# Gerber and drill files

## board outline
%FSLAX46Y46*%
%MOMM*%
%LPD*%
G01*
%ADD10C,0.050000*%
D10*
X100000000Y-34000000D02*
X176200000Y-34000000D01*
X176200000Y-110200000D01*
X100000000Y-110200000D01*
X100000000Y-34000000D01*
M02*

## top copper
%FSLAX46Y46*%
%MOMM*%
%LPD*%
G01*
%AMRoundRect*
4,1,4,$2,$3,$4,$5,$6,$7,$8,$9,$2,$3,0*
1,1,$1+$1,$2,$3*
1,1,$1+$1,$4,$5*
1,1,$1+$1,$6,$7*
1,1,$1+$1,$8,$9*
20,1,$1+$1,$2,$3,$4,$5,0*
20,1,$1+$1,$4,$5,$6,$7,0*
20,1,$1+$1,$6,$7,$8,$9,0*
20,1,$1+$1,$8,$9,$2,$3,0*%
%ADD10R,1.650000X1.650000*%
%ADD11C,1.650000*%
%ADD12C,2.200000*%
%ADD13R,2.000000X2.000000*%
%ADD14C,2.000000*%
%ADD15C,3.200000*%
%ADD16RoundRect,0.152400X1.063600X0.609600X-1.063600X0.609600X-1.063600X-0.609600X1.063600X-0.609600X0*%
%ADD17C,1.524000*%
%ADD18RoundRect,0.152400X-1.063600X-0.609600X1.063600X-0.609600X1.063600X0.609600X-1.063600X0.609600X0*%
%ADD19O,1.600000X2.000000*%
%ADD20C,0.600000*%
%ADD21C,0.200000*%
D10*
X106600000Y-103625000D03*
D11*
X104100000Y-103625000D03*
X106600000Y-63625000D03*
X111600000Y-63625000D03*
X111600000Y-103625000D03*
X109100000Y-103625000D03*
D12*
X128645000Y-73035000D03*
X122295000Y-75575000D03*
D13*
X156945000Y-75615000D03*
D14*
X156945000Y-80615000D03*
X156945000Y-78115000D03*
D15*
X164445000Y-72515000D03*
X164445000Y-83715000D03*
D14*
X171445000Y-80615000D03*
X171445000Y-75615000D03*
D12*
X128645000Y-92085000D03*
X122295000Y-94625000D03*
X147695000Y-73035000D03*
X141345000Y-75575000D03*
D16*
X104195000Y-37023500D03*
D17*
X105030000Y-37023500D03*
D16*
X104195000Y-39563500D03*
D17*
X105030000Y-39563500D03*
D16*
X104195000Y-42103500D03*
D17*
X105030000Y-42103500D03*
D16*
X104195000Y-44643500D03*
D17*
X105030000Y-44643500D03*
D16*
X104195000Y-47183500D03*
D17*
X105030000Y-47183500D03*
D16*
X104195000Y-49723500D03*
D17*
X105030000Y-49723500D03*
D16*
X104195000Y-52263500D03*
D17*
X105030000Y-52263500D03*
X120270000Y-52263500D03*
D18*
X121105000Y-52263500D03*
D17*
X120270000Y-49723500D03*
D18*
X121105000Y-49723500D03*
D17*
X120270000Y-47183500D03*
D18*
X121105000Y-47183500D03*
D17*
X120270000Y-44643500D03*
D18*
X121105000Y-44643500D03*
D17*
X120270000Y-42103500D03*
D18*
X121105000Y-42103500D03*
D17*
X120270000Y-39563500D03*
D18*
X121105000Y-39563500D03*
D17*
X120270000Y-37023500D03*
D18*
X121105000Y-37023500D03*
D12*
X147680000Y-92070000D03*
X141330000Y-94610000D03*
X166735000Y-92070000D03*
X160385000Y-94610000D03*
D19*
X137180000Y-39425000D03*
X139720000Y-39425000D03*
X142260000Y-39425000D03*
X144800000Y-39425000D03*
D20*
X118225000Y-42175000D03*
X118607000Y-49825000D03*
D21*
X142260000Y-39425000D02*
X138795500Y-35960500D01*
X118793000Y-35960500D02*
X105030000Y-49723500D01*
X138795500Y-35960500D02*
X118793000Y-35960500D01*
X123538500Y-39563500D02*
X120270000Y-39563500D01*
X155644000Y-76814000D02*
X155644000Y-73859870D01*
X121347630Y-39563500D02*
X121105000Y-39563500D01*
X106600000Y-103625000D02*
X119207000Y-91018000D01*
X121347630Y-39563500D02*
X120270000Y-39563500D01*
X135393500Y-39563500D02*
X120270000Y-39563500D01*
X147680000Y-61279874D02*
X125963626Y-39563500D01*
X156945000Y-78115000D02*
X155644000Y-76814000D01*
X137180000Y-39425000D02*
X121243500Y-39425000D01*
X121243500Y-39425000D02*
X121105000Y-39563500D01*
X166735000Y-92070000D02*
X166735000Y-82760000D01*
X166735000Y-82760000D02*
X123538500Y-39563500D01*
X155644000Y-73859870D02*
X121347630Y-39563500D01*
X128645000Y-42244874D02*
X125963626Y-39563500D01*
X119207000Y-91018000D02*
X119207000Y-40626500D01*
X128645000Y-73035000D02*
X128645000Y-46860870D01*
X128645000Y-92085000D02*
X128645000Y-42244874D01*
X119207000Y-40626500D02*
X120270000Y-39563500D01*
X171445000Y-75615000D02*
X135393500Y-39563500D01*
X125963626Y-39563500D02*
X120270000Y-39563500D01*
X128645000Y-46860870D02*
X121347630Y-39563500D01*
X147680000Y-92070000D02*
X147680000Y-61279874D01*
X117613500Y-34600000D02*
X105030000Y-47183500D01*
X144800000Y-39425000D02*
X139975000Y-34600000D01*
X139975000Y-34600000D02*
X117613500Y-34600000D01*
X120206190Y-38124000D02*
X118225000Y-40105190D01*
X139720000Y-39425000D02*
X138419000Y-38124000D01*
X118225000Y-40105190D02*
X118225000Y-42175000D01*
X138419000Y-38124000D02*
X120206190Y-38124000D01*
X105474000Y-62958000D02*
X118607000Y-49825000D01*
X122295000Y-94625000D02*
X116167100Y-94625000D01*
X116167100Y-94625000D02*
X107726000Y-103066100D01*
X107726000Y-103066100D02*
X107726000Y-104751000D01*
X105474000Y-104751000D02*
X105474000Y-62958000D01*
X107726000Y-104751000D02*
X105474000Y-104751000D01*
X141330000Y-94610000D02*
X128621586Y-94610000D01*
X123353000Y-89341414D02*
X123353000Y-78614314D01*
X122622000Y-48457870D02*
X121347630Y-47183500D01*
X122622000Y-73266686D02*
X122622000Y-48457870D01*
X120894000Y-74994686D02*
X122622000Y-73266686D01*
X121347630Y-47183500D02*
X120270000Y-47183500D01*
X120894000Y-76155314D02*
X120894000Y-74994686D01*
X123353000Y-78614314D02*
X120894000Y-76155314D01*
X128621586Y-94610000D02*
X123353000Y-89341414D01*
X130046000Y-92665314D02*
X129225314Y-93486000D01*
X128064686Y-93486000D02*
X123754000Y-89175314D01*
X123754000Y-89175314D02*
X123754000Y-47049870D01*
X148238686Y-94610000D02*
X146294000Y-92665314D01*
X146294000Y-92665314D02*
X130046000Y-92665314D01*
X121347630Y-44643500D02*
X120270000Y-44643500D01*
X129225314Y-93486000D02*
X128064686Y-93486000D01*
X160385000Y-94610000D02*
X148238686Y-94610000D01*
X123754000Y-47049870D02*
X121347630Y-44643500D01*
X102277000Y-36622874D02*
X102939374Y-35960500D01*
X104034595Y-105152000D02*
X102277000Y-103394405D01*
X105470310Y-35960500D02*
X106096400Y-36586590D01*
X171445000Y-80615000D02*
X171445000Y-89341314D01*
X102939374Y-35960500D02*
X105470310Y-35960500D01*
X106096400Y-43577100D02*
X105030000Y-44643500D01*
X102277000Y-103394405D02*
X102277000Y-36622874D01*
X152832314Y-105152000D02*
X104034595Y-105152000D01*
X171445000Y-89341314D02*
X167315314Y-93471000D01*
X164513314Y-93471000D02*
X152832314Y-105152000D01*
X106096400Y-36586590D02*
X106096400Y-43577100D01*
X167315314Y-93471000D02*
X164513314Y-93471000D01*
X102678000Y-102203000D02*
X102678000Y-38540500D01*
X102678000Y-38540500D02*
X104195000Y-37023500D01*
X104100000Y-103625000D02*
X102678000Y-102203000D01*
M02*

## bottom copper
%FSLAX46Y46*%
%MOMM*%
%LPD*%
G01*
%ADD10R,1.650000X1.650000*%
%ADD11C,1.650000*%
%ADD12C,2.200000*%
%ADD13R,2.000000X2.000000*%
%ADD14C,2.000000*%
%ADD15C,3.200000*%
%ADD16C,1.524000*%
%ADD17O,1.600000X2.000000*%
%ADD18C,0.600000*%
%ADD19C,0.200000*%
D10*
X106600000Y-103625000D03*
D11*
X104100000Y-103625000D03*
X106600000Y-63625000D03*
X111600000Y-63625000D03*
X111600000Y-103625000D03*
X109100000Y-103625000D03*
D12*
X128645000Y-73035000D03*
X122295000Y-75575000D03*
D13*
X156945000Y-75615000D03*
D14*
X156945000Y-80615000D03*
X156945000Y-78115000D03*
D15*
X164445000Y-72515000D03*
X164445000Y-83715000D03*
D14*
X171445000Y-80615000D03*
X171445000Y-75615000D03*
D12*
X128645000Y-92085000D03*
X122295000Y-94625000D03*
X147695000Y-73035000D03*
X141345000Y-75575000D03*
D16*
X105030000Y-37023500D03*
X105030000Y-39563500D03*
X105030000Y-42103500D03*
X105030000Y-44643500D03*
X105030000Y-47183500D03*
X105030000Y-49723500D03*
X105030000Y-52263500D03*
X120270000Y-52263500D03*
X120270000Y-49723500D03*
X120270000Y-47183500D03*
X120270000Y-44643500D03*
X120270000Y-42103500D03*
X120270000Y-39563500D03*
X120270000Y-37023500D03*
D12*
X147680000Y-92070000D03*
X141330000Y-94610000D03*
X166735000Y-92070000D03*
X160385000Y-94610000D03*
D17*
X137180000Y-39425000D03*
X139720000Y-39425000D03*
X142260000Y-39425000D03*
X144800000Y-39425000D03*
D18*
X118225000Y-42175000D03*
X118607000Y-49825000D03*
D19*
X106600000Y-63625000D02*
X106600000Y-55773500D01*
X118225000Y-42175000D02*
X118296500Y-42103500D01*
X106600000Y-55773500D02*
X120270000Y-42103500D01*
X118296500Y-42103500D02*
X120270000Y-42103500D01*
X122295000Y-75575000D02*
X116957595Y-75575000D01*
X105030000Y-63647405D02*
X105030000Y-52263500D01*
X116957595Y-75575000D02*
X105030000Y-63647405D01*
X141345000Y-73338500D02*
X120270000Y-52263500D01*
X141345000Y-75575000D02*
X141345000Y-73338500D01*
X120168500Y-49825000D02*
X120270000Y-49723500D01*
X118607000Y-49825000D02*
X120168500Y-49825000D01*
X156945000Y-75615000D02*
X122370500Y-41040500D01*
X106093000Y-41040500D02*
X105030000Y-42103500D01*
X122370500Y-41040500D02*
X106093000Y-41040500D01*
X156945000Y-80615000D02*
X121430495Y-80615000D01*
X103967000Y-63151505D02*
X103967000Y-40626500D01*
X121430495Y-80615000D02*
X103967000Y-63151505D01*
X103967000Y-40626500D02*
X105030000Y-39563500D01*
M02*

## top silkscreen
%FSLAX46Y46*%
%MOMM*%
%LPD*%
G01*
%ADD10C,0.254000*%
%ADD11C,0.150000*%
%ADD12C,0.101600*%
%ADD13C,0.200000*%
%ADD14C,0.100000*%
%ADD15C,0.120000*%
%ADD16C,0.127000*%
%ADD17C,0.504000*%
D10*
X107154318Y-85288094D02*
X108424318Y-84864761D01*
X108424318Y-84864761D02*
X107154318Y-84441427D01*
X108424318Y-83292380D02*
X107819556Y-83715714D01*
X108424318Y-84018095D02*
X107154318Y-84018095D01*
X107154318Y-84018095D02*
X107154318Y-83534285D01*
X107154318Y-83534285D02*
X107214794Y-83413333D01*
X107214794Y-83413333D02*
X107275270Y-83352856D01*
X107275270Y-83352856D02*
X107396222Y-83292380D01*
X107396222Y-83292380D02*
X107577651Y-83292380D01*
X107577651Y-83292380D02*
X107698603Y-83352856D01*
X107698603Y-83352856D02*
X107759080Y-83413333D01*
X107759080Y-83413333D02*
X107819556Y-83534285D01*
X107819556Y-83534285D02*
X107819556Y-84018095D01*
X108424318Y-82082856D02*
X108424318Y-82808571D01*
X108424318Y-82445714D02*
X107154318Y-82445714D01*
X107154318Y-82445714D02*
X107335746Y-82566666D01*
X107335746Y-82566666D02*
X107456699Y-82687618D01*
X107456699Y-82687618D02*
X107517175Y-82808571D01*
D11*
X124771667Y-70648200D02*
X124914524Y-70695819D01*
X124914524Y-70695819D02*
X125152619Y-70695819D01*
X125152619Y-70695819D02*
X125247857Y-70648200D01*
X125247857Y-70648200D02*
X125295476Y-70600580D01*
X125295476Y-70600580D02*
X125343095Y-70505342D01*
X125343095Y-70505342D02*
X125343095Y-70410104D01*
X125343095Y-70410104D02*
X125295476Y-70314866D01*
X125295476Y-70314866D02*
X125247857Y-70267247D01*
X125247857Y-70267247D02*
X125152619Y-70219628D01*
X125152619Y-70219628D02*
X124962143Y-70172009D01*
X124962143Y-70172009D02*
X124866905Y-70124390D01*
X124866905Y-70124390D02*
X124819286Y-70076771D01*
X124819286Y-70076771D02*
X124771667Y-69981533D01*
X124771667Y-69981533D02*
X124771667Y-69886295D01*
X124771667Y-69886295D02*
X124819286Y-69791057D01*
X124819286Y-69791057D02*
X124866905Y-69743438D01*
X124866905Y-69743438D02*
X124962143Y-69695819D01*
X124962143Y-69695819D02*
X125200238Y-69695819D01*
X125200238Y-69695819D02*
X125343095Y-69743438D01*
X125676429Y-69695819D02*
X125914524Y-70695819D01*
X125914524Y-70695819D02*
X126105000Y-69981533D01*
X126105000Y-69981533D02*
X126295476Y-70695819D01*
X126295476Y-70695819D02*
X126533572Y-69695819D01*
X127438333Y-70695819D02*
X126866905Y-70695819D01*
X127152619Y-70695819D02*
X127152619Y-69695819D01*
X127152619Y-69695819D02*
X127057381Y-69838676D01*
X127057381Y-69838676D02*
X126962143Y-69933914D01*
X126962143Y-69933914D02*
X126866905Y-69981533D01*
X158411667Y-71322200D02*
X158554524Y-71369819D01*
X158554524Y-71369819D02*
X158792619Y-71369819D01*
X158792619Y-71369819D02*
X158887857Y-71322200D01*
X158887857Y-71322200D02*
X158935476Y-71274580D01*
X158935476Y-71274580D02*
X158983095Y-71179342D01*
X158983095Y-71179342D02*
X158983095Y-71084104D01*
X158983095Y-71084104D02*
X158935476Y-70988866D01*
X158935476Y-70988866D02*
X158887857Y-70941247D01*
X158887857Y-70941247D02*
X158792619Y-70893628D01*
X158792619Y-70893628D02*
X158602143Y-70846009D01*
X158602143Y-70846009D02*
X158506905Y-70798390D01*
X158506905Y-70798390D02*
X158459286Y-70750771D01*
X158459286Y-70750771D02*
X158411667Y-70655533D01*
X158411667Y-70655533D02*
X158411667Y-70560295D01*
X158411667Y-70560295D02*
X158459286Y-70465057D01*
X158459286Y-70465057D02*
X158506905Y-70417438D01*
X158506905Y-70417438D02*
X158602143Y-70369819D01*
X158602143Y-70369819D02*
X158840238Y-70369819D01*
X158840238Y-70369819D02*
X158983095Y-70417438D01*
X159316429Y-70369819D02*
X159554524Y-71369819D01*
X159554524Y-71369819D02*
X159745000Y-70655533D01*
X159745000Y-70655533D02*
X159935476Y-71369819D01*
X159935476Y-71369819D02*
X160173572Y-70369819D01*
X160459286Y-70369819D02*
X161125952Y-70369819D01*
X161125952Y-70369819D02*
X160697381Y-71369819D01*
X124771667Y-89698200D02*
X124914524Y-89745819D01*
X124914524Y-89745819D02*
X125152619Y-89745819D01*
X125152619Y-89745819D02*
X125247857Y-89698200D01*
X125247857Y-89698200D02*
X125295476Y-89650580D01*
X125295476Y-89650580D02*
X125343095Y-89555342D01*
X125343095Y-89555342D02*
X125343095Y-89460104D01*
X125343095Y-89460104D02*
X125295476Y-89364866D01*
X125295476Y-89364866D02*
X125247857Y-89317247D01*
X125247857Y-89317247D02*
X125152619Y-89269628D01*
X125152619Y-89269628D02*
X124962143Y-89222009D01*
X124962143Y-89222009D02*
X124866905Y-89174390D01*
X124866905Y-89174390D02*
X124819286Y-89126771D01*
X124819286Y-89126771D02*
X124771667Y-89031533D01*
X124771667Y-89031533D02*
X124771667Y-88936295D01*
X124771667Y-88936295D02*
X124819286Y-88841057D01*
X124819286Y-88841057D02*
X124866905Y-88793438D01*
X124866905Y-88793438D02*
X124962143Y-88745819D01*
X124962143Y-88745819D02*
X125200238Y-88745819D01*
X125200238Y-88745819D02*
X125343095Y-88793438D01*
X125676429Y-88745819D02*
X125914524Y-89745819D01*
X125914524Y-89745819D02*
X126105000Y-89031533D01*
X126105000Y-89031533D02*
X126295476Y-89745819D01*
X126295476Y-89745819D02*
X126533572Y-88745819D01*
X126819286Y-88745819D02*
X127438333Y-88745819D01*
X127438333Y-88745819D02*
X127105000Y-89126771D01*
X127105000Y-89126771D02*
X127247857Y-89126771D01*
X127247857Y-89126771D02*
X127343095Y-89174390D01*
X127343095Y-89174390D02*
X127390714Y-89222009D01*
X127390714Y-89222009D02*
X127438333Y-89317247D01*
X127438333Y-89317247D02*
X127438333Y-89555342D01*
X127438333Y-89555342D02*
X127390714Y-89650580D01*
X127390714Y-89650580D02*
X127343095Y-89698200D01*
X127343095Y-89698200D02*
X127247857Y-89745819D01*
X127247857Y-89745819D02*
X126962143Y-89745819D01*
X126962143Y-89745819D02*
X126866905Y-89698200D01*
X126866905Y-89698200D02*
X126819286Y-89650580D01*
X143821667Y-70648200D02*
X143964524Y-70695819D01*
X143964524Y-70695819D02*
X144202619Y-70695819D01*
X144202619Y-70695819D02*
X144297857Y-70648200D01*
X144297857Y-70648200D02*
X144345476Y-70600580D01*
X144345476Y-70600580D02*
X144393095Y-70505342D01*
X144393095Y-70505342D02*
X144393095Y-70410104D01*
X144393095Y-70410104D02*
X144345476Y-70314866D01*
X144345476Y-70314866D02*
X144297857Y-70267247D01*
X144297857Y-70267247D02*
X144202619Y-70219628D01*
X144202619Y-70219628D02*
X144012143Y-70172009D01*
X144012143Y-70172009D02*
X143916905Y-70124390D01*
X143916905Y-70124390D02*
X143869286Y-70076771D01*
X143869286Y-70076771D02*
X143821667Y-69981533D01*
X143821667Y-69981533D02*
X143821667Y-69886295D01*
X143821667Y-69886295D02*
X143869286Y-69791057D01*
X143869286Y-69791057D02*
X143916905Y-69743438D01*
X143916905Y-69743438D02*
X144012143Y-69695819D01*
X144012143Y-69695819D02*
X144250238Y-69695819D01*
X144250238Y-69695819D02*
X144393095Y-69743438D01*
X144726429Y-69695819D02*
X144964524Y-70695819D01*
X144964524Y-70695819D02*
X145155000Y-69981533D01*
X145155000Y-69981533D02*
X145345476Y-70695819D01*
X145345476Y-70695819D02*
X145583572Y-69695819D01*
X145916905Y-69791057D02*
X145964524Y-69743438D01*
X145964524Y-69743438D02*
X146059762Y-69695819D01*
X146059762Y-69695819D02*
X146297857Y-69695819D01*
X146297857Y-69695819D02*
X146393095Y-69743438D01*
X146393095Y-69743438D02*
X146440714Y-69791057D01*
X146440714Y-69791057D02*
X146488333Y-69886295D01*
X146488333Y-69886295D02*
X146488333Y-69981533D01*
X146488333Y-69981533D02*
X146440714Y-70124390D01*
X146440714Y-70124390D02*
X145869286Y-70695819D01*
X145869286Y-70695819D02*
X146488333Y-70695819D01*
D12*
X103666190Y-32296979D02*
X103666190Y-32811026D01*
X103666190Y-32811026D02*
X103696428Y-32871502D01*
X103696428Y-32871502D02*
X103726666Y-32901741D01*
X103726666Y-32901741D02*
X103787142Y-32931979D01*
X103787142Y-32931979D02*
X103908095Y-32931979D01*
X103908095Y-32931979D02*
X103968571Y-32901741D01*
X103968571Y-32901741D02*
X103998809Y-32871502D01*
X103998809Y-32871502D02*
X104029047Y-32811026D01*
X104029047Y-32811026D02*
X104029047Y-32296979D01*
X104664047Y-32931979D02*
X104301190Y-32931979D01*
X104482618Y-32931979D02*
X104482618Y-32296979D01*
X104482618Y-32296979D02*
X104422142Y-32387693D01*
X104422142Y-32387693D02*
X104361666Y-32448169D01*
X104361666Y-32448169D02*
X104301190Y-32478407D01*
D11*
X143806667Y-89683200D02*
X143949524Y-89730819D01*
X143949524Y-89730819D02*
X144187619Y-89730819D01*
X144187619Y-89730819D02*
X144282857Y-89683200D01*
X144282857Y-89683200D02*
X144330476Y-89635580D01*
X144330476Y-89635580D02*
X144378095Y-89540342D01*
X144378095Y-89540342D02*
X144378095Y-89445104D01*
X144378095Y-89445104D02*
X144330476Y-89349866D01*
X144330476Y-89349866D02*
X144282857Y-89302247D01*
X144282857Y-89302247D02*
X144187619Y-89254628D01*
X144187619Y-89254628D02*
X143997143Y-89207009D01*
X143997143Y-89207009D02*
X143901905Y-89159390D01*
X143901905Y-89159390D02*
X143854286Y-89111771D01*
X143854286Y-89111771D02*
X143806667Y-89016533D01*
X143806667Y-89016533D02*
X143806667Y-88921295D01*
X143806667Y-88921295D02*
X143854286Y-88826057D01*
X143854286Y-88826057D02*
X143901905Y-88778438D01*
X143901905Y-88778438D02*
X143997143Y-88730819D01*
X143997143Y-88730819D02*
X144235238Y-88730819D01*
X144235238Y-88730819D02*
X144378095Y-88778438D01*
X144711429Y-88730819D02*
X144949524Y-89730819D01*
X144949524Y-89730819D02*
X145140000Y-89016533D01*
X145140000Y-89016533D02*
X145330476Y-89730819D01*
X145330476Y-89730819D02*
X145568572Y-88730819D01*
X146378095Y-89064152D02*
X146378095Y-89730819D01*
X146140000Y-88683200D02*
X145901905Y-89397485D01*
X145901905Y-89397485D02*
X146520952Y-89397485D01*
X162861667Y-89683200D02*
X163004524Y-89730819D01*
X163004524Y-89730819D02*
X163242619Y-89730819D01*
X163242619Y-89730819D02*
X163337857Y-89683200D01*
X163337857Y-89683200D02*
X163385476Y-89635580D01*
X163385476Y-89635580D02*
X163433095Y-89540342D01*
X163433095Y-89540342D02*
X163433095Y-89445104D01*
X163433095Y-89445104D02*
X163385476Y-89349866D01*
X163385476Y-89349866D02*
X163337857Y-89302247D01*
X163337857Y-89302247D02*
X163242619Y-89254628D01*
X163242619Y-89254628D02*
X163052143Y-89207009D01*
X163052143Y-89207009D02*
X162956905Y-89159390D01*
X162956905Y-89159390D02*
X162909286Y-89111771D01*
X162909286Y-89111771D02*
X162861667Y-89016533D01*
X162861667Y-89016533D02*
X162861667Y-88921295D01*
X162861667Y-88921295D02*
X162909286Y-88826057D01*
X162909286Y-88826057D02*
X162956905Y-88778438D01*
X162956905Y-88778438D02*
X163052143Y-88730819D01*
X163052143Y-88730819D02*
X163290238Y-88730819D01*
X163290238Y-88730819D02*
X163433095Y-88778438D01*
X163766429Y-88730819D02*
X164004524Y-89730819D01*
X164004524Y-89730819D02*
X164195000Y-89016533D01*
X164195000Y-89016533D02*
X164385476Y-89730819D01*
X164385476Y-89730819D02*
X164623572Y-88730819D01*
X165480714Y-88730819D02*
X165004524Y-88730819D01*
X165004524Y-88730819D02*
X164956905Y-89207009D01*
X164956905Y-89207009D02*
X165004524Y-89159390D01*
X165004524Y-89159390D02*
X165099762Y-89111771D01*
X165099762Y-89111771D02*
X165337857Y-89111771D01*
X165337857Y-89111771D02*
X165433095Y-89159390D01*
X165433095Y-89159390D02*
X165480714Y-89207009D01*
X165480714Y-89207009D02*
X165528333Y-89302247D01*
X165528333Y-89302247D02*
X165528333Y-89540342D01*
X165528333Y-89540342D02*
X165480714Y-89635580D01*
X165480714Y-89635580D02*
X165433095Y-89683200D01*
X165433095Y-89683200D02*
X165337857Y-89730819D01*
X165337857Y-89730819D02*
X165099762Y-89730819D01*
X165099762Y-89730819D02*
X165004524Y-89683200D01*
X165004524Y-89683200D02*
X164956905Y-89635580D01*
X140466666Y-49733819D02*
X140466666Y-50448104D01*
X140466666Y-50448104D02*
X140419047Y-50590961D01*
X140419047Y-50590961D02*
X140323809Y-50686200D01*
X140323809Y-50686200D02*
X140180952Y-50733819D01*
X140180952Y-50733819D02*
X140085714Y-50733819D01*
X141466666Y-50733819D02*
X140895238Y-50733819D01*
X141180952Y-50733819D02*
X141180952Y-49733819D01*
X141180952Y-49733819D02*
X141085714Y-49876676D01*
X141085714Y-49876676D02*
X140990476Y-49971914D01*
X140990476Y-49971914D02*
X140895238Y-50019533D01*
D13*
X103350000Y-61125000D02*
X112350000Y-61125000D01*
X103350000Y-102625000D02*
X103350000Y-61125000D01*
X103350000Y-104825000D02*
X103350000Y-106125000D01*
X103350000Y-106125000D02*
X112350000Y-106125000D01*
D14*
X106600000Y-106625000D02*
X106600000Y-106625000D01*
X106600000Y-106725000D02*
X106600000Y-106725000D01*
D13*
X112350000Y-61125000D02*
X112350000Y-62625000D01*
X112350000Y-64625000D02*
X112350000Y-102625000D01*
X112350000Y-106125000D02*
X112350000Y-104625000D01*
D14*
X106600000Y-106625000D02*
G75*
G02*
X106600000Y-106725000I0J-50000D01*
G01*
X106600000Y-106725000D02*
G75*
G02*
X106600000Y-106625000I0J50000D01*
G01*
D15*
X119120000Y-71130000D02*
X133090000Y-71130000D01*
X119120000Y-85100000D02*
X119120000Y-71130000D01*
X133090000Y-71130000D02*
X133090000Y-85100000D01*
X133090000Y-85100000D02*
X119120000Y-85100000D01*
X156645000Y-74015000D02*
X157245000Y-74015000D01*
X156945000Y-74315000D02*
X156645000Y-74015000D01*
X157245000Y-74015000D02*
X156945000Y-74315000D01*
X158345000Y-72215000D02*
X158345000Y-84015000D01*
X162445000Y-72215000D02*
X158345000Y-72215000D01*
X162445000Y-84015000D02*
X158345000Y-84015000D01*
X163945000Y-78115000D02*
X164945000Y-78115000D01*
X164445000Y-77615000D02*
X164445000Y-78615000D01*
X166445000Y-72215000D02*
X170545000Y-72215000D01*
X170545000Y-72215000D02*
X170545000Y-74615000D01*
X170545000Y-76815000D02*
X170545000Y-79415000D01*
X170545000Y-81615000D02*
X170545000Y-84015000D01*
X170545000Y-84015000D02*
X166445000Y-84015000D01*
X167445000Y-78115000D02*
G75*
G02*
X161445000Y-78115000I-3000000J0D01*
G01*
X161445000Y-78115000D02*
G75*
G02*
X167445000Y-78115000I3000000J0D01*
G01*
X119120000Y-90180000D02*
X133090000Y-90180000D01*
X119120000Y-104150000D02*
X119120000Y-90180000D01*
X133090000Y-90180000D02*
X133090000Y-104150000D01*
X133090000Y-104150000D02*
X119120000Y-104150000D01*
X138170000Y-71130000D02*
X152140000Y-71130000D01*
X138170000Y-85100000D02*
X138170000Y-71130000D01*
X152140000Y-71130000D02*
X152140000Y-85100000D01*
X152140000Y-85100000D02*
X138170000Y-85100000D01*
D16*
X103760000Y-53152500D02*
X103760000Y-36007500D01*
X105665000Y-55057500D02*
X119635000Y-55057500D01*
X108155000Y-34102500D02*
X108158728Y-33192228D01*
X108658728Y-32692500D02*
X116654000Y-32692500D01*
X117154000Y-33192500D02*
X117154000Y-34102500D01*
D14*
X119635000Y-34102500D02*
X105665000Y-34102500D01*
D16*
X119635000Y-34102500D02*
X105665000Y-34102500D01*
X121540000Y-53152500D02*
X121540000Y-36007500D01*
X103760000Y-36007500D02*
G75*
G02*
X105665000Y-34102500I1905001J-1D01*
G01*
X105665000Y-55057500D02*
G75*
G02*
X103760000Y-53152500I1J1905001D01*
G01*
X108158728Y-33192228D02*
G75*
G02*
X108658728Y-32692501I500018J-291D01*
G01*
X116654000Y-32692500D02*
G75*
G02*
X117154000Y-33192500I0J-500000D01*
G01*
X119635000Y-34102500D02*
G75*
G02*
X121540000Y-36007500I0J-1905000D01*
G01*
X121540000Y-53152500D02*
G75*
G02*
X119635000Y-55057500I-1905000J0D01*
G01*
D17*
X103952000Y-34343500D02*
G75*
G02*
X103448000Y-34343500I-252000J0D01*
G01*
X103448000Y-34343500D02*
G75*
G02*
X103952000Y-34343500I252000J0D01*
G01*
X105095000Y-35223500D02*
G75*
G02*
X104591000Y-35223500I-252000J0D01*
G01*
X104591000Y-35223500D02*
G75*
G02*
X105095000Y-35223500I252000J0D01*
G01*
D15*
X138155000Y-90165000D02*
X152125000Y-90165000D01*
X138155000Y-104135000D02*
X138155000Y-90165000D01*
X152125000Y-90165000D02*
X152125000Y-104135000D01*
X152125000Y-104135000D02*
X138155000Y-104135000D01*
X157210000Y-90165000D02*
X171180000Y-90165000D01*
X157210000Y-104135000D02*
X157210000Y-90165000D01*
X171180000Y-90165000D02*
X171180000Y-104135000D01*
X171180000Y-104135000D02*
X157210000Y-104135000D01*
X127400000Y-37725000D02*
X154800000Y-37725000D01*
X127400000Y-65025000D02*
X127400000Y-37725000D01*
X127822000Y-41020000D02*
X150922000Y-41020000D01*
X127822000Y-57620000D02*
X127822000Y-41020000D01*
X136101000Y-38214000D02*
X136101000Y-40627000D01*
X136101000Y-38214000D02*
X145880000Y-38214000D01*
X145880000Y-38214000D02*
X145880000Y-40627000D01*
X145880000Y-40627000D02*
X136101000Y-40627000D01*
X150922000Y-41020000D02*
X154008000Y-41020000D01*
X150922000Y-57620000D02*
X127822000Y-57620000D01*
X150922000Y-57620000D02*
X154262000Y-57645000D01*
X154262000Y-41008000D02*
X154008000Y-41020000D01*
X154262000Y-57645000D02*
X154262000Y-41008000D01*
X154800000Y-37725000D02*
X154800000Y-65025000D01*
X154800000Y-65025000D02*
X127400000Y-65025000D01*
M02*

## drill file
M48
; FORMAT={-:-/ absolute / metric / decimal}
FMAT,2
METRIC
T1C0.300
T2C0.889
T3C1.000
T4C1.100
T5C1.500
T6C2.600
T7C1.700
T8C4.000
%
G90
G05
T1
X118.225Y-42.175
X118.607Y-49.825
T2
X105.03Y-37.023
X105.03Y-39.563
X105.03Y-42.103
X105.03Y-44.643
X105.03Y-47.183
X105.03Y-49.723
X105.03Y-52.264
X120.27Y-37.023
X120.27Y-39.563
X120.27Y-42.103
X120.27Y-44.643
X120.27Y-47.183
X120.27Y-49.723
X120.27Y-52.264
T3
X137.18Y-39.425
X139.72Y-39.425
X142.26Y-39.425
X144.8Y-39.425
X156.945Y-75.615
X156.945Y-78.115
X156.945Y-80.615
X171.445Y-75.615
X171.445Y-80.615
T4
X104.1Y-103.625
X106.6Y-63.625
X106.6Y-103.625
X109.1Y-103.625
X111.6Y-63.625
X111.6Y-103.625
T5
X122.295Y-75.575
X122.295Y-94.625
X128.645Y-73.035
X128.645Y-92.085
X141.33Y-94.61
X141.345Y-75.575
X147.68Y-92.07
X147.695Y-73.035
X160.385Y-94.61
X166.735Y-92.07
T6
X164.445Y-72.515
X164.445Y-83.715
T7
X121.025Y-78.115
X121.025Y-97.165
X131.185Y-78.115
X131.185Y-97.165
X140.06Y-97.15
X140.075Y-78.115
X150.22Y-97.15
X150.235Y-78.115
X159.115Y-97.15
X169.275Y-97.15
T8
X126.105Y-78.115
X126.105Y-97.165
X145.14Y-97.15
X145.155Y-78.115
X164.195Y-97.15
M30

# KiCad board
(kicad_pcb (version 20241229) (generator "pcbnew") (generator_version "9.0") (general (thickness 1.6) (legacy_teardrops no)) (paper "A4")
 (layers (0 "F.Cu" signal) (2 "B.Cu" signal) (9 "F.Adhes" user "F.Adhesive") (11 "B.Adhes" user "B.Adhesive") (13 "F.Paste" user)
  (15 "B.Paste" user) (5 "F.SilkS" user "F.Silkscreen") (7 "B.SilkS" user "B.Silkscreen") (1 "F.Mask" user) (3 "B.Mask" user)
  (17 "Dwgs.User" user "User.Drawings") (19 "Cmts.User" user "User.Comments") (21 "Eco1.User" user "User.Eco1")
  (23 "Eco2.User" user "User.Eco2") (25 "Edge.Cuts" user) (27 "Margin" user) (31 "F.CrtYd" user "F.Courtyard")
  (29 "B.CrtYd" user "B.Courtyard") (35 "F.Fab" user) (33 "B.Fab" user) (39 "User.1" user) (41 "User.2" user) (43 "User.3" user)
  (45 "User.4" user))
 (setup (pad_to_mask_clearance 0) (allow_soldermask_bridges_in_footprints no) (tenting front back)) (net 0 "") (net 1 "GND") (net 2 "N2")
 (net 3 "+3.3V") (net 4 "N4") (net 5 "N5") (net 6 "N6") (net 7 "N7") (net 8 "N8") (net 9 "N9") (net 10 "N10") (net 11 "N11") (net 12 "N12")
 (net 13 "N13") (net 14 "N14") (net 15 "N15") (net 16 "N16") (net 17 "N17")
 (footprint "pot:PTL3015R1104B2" (layer "F.Cu") (at 106.6 103.625 90)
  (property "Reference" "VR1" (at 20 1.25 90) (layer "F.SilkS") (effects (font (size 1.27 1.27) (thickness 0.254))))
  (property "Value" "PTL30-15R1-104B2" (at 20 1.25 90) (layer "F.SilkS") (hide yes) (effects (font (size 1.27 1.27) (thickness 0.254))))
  (fp_line (start 42.5 -3.25) (end 42.5 5.75) (stroke (width 0.2) (type solid)) (layer "F.SilkS"))
  (fp_line (start 1 -3.25) (end 42.5 -3.25) (stroke (width 0.2) (type solid)) (layer "F.SilkS"))
  (fp_line (start -1.2 -3.25) (end -2.5 -3.25) (stroke (width 0.2) (type solid)) (layer "F.SilkS"))
  (fp_line (start -2.5 -3.25) (end -2.5 5.75) (stroke (width 0.2) (type solid)) (layer "F.SilkS"))
  (fp_line (start -3 0) (end -3 0) (stroke (width 0.1) (type solid)) (layer "F.SilkS"))
  (fp_line (start -3.1 0) (end -3.1 0) (stroke (width 0.1) (type solid)) (layer "F.SilkS"))
  (fp_line (start 42.5 5.75) (end 41 5.75) (stroke (width 0.2) (type solid)) (layer "F.SilkS"))
  (fp_line (start 39 5.75) (end 1 5.75) (stroke (width 0.2) (type solid)) (layer "F.SilkS"))
  (fp_line (start -2.5 5.75) (end -1 5.75) (stroke (width 0.2) (type solid)) (layer "F.SilkS"))
  (fp_arc (start -3 0) (mid -3.05 0.05) (end -3.1 0) (stroke (width 0.1) (type solid)) (layer "F.SilkS"))
  (fp_arc (start -3.1 0) (mid -3.05 -0.05) (end -3 0) (stroke (width 0.1) (type solid)) (layer "F.SilkS"))
  (pad "1" thru_hole rect (at 0 0 90) (size 1.65 1.65) (drill 1.1) (layers "*.Cu" "*.Mask") (remove_unused_layers no) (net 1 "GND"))
  (pad "2" thru_hole circle (at 0 -2.5 90) (size 1.65 1.65) (drill 1.1) (layers "*.Cu" "*.Mask") (remove_unused_layers no) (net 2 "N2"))
  (pad "3" thru_hole circle (at 40 0 90) (size 1.65 1.65) (drill 1.1) (layers "*.Cu" "*.Mask") (remove_unused_layers no) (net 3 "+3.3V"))
  (pad "B1" thru_hole circle (at 40 5 90) (size 1.65 1.65) (drill 1.1) (layers "*.Cu" "*.Mask") (remove_unused_layers no) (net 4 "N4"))
  (pad "E1" thru_hole circle (at 0 5 90) (size 1.65 1.65) (drill 1.1) (layers "*.Cu" "*.Mask") (remove_unused_layers no) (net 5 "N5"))
  (pad "L1" thru_hole circle (at 0 2.5 90) (size 1.65 1.65) (drill 1.1) (layers "*.Cu" "*.Mask") (remove_unused_layers no) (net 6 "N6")))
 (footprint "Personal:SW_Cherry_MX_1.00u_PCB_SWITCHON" (layer "F.Cu") (at 128.645 73.035)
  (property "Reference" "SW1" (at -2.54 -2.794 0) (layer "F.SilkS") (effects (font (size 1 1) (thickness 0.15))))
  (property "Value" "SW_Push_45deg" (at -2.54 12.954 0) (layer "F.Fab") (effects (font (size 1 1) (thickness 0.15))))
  (fp_line (start -9.525 -1.905) (end 4.445 -1.905) (stroke (width 0.12) (type solid)) (layer "F.SilkS"))
  (fp_line (start -9.525 12.065) (end -9.525 -1.905) (stroke (width 0.12) (type solid)) (layer "F.SilkS"))
  (fp_line (start 4.445 -1.905) (end 4.445 12.065) (stroke (width 0.12) (type solid)) (layer "F.SilkS"))
  (fp_line (start 4.445 12.065) (end -9.525 12.065) (stroke (width 0.12) (type solid)) (layer "F.SilkS"))
  (pad "" np_thru_hole circle (at -7.62 5.08) (size 1.7 1.7) (drill 1.7) (layers "*.Cu" "*.Mask"))
  (pad "" np_thru_hole circle (at -2.54 5.08) (size 4 4) (drill 4) (layers "*.Cu" "*.Mask"))
  (pad "" np_thru_hole circle (at 2.54 5.08) (size 1.7 1.7) (drill 1.7) (layers "*.Cu" "*.Mask"))
  (pad "1" thru_hole circle (at 0 0) (size 2.2 2.2) (drill 1.5) (layers "*.Cu" "*.Mask") (remove_unused_layers no) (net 1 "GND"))
  (pad "2" thru_hole circle (at -6.35 2.54) (size 2.2 2.2) (drill 1.5) (layers "*.Cu" "*.Mask") (remove_unused_layers no) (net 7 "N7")))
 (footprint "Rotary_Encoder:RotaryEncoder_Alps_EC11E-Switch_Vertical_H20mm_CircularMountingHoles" (layer "F.Cu") (at 156.945 75.615)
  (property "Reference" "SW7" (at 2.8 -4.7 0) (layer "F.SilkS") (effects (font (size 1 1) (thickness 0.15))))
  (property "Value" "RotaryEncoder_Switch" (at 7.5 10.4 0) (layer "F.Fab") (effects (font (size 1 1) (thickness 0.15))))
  (fp_line (start -0.3 -1.6) (end 0.3 -1.6) (stroke (width 0.12) (type solid)) (layer "F.SilkS"))
  (fp_line (start 0 -1.3) (end -0.3 -1.6) (stroke (width 0.12) (type solid)) (layer "F.SilkS"))
  (fp_line (start 0.3 -1.6) (end 0 -1.3) (stroke (width 0.12) (type solid)) (layer "F.SilkS"))
  (fp_line (start 1.4 -3.4) (end 1.4 8.4) (stroke (width 0.12) (type solid)) (layer "F.SilkS"))
  (fp_line (start 5.5 -3.4) (end 1.4 -3.4) (stroke (width 0.12) (type solid)) (layer "F.SilkS"))
  (fp_line (start 5.5 8.4) (end 1.4 8.4) (stroke (width 0.12) (type solid)) (layer "F.SilkS"))
  (fp_line (start 7 2.5) (end 8 2.5) (stroke (width 0.12) (type solid)) (layer "F.SilkS"))
  (fp_line (start 7.5 2) (end 7.5 3) (stroke (width 0.12) (type solid)) (layer "F.SilkS"))
  (fp_line (start 9.5 -3.4) (end 13.6 -3.4) (stroke (width 0.12) (type solid)) (layer "F.SilkS"))
  (fp_line (start 13.6 -3.4) (end 13.6 -1) (stroke (width 0.12) (type solid)) (layer "F.SilkS"))
  (fp_line (start 13.6 1.2) (end 13.6 3.8) (stroke (width 0.12) (type solid)) (layer "F.SilkS"))
  (fp_line (start 13.6 6) (end 13.6 8.4) (stroke (width 0.12) (type solid)) (layer "F.SilkS"))
  (fp_line (start 13.6 8.4) (end 9.5 8.4) (stroke (width 0.12) (type solid)) (layer "F.SilkS"))
  (fp_circle (center 7.5 2.5) (end 10.5 2.5) (stroke (width 0.12) (type solid)) (fill no) (layer "F.SilkS"))
  (pad "A" thru_hole rect (at 0 0) (size 2 2) (drill 1) (layers "*.Cu" "*.Mask") (remove_unused_layers no) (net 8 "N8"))
  (pad "B" thru_hole circle (at 0 5) (size 2 2) (drill 1) (layers "*.Cu" "*.Mask") (remove_unused_layers no) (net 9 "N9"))
  (pad "C" thru_hole circle (at 0 2.5) (size 2 2) (drill 1) (layers "*.Cu" "*.Mask") (remove_unused_layers no) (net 1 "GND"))
  (pad "MP" thru_hole circle (at 7.5 -3.1) (size 3.2 3.2) (drill 2.6) (layers "*.Cu" "*.Mask") (remove_unused_layers no))
  (pad "MP" thru_hole circle (at 7.5 8.1) (size 3.2 3.2) (drill 2.6) (layers "*.Cu" "*.Mask") (remove_unused_layers no))
  (pad "S1" thru_hole circle (at 14.5 5) (size 2 2) (drill 1) (layers "*.Cu" "*.Mask") (remove_unused_layers no) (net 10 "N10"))
  (pad "S2" thru_hole circle (at 14.5 0) (size 2 2) (drill 1) (layers "*.Cu" "*.Mask") (remove_unused_layers no) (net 1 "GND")))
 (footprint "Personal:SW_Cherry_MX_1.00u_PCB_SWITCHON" (layer "F.Cu") (at 128.645 92.085)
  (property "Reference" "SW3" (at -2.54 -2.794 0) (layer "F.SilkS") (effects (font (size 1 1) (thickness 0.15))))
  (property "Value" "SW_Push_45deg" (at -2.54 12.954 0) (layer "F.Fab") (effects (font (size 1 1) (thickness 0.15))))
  (fp_line (start -9.525 -1.905) (end 4.445 -1.905) (stroke (width 0.12) (type solid)) (layer "F.SilkS"))
  (fp_line (start -9.525 12.065) (end -9.525 -1.905) (stroke (width 0.12) (type solid)) (layer "F.SilkS"))
  (fp_line (start 4.445 -1.905) (end 4.445 12.065) (stroke (width 0.12) (type solid)) (layer "F.SilkS"))
  (fp_line (start 4.445 12.065) (end -9.525 12.065) (stroke (width 0.12) (type solid)) (layer "F.SilkS"))
  (pad "" np_thru_hole circle (at -7.62 5.08) (size 1.7 1.7) (drill 1.7) (layers "*.Cu" "*.Mask"))
  (pad "" np_thru_hole circle (at -2.54 5.08) (size 4 4) (drill 4) (layers "*.Cu" "*.Mask"))
  (pad "" np_thru_hole circle (at 2.54 5.08) (size 1.7 1.7) (drill 1.7) (layers "*.Cu" "*.Mask"))
  (pad "1" thru_hole circle (at 0 0) (size 2.2 2.2) (drill 1.5) (layers "*.Cu" "*.Mask") (remove_unused_layers no) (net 1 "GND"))
  (pad "2" thru_hole circle (at -6.35 2.54) (size 2.2 2.2) (drill 1.5) (layers "*.Cu" "*.Mask") (remove_unused_layers no) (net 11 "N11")))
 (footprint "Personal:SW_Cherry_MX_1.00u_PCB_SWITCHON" (layer "F.Cu") (at 147.695 73.035)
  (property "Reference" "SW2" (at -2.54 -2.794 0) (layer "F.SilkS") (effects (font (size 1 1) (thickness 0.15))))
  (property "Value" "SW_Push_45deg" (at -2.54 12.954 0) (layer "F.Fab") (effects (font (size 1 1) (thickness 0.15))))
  (fp_line (start -9.525 -1.905) (end 4.445 -1.905) (stroke (width 0.12) (type solid)) (layer "F.SilkS"))
  (fp_line (start -9.525 12.065) (end -9.525 -1.905) (stroke (width 0.12) (type solid)) (layer "F.SilkS"))
  (fp_line (start 4.445 -1.905) (end 4.445 12.065) (stroke (width 0.12) (type solid)) (layer "F.SilkS"))
  (fp_line (start 4.445 12.065) (end -9.525 12.065) (stroke (width 0.12) (type solid)) (layer "F.SilkS"))
  (pad "" np_thru_hole circle (at -7.62 5.08) (size 1.7 1.7) (drill 1.7) (layers "*.Cu" "*.Mask"))
  (pad "" np_thru_hole circle (at -2.54 5.08) (size 4 4) (drill 4) (layers "*.Cu" "*.Mask"))
  (pad "" np_thru_hole circle (at 2.54 5.08) (size 1.7 1.7) (drill 1.7) (layers "*.Cu" "*.Mask"))
  (pad "1" thru_hole circle (at 0 0) (size 2.2 2.2) (drill 1.5) (layers "*.Cu" "*.Mask") (remove_unused_layers no) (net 1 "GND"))
  (pad "2" thru_hole circle (at -6.35 2.54) (size 2.2 2.2) (drill 1.5) (layers "*.Cu" "*.Mask") (remove_unused_layers no) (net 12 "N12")))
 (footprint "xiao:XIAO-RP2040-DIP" (layer "F.Cu") (at 112.65 44.6435)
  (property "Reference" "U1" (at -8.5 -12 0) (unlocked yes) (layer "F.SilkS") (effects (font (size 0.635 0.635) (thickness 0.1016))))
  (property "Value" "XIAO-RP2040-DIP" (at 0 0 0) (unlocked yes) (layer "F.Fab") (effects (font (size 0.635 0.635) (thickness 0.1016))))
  (fp_line (start -8.89 8.509) (end -8.89 -8.636) (stroke (width 0.127) (type solid)) (layer "F.SilkS"))
  (fp_line (start -6.985 10.414) (end 6.985 10.414) (stroke (width 0.127) (type solid)) (layer "F.SilkS"))
  (fp_line (start -4.495 -10.541) (end -4.491272 -11.451272) (stroke (width 0.127) (type solid)) (layer "F.SilkS"))
  (fp_line (start -3.991272 -11.951) (end 4.004 -11.951) (stroke (width 0.127) (type solid)) (layer "F.SilkS"))
  (fp_line (start 4.504 -11.451) (end 4.504 -10.541) (stroke (width 0.127) (type solid)) (layer "F.SilkS"))
  (fp_line (start 6.985 -10.541) (end -6.985 -10.541) (stroke (width 0.1) (type solid)) (layer "F.SilkS"))
  (fp_line (start 6.985 -10.541) (end -6.985 -10.541) (stroke (width 0.127) (type solid)) (layer "F.SilkS"))
  (fp_line (start 8.89 8.509) (end 8.89 -8.636) (stroke (width 0.127) (type solid)) (layer "F.SilkS"))
  (fp_arc (start -8.89 -8.636) (mid -8.332038 -9.983038) (end -6.985 -10.541) (stroke (width 0.127) (type solid)) (layer "F.SilkS"))
  (fp_arc (start -6.985 10.414) (mid -8.332038 9.856038) (end -8.89 8.509) (stroke (width 0.127) (type solid)) (layer "F.SilkS"))
  (fp_arc (start -4.491272 -11.451272) (mid -4.344728 -11.80464) (end -3.991272 -11.951) (stroke (width 0.127) (type default))
   (layer "F.SilkS"))
  (fp_arc (start 4.004 -11.951) (mid 4.357553 -11.804553) (end 4.504 -11.451) (stroke (width 0.127) (type default)) (layer "F.SilkS"))
  (fp_arc (start 6.985 -10.541) (mid 8.332038 -9.983038) (end 8.89 -8.636) (stroke (width 0.127) (type solid)) (layer "F.SilkS"))
  (fp_arc (start 8.89 8.509) (mid 8.332038 9.856038) (end 6.985 10.414) (stroke (width 0.127) (type solid)) (layer "F.SilkS"))
  (fp_circle (center -8.95 -10.3) (end -8.95 -10.554) (stroke (width 0.5) (type solid)) (fill yes) (layer "F.SilkS"))
  (fp_circle (center -7.807 -9.42) (end -7.807 -9.674) (stroke (width 0.5) (type solid)) (fill yes) (layer "F.SilkS"))
  (pad "1" smd roundrect (at -8.455 -7.62 180) (size 2.432 1.524) (layers "F.Cu" "F.Mask") (roundrect_rratio 0.1) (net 2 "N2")
   (thermal_bridge_angle 45))
  (pad "1" thru_hole circle (at -7.62 -7.62 180) (size 1.524 1.524) (drill 0.889) (layers "*.Cu" "*.Mask") (remove_unused_layers no)
   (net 2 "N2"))
  (pad "2" smd roundrect (at -8.455 -5.08 180) (size 2.432 1.524) (layers "F.Cu" "F.Mask") (roundrect_rratio 0.1) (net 9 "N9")
   (thermal_bridge_angle 45))
  (pad "2" thru_hole circle (at -7.62 -5.08 180) (size 1.524 1.524) (drill 0.889) (layers "*.Cu" "*.Mask") (remove_unused_layers no)
   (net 9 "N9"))
  (pad "3" smd roundrect (at -8.455 -2.54 180) (size 2.432 1.524) (layers "F.Cu" "F.Mask") (roundrect_rratio 0.1) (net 8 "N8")
   (thermal_bridge_angle 45))
  (pad "3" thru_hole circle (at -7.62 -2.54 180) (size 1.524 1.524) (drill 0.889) (layers "*.Cu" "*.Mask") (remove_unused_layers no)
   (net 8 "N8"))
  (pad "4" smd roundrect (at -8.455 0 180) (size 2.432 1.524) (layers "F.Cu" "F.Mask") (roundrect_rratio 0.1) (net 10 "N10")
   (thermal_bridge_angle 45))
  (pad "4" thru_hole circle (at -7.62 0 180) (size 1.524 1.524) (drill 0.889) (layers "*.Cu" "*.Mask") (remove_unused_layers no)
   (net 10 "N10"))
  (pad "5" smd roundrect (at -8.455 2.54 180) (size 2.432 1.524) (layers "F.Cu" "F.Mask") (roundrect_rratio 0.1) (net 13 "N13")
   (thermal_bridge_angle 45))
  (pad "5" thru_hole circle (at -7.62 2.54 180) (size 1.524 1.524) (drill 0.889) (layers "*.Cu" "*.Mask") (remove_unused_layers no)
   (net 13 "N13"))
  (pad "6" smd roundrect (at -8.455 5.08 180) (size 2.432 1.524) (layers "F.Cu" "F.Mask") (roundrect_rratio 0.1) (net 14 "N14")
   (thermal_bridge_angle 45))
  (pad "6" thru_hole circle (at -7.62 5.08 180) (size 1.524 1.524) (drill 0.889) (layers "*.Cu" "*.Mask") (remove_unused_layers no)
   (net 14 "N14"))
  (pad "7" smd roundrect (at -8.455 7.62 180) (size 2.432 1.524) (layers "F.Cu" "F.Mask") (roundrect_rratio 0.1) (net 7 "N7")
   (thermal_bridge_angle 45))
  (pad "7" thru_hole circle (at -7.62 7.62 180) (size 1.524 1.524) (drill 0.889) (layers "*.Cu" "*.Mask") (remove_unused_layers no)
   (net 7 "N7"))
  (pad "8" thru_hole circle (at 7.62 7.62) (size 1.524 1.524) (drill 0.889) (layers "*.Cu" "*.Mask") (remove_unused_layers no)
   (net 12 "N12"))
  (pad "8" smd roundrect (at 8.455 7.62) (size 2.432 1.524) (layers "F.Cu" "F.Mask") (roundrect_rratio 0.1) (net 12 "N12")
   (thermal_bridge_angle 45))
  (pad "9" thru_hole circle (at 7.62 5.08) (size 1.524 1.524) (drill 0.889) (layers "*.Cu" "*.Mask") (remove_unused_layers no)
   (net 11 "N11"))
  (pad "9" smd roundrect (at 8.455 5.08) (size 2.432 1.524) (layers "F.Cu" "F.Mask") (roundrect_rratio 0.1) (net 11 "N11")
   (thermal_bridge_angle 45))
  (pad "10" thru_hole circle (at 7.62 2.54) (size 1.524 1.524) (drill 0.889) (layers "*.Cu" "*.Mask") (remove_unused_layers no)
   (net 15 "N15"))
  (pad "10" smd roundrect (at 8.455 2.54) (size 2.432 1.524) (layers "F.Cu" "F.Mask") (roundrect_rratio 0.1) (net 15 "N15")
   (thermal_bridge_angle 45))
  (pad "11" thru_hole circle (at 7.62 0) (size 1.524 1.524) (drill 0.889) (layers "*.Cu" "*.Mask") (remove_unused_layers no) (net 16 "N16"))
  (pad "11" smd roundrect (at 8.455 0) (size 2.432 1.524) (layers "F.Cu" "F.Mask") (roundrect_rratio 0.1) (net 16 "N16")
   (thermal_bridge_angle 45))
  (pad "12" thru_hole circle (at 7.62 -2.54) (size 1.524 1.524) (drill 0.889) (layers "*.Cu" "*.Mask") (remove_unused_layers no)
   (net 3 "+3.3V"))
  (pad "12" smd roundrect (at 8.455 -2.54) (size 2.432 1.524) (layers "F.Cu" "F.Mask") (roundrect_rratio 0.1) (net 3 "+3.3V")
   (thermal_bridge_angle 45))
  (pad "13" thru_hole circle (at 7.62 -5.08) (size 1.524 1.524) (drill 0.889) (layers "*.Cu" "*.Mask") (remove_unused_layers no)
   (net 1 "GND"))
  (pad "13" smd roundrect (at 8.455 -5.08) (size 2.432 1.524) (layers "F.Cu" "F.Mask") (roundrect_rratio 0.1) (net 1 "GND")
   (thermal_bridge_angle 45))
  (pad "14" thru_hole circle (at 7.62 -7.62) (size 1.524 1.524) (drill 0.889) (layers "*.Cu" "*.Mask") (remove_unused_layers no)
   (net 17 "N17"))
  (pad "14" smd roundrect (at 8.455 -7.62) (size 2.432 1.524) (layers "F.Cu" "F.Mask") (roundrect_rratio 0.1) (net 17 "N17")
   (thermal_bridge_angle 45)))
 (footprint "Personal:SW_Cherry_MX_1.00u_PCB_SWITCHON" (layer "F.Cu") (at 147.68 92.07)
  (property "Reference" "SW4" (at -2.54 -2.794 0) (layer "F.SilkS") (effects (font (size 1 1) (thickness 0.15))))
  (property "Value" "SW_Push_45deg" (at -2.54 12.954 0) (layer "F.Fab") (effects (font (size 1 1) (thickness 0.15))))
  (fp_line (start -9.525 -1.905) (end 4.445 -1.905) (stroke (width 0.12) (type solid)) (layer "F.SilkS"))
  (fp_line (start -9.525 12.065) (end -9.525 -1.905) (stroke (width 0.12) (type solid)) (layer "F.SilkS"))
  (fp_line (start 4.445 -1.905) (end 4.445 12.065) (stroke (width 0.12) (type solid)) (layer "F.SilkS"))
  (fp_line (start 4.445 12.065) (end -9.525 12.065) (stroke (width 0.12) (type solid)) (layer "F.SilkS"))
  (pad "" np_thru_hole circle (at -7.62 5.08) (size 1.7 1.7) (drill 1.7) (layers "*.Cu" "*.Mask"))
  (pad "" np_thru_hole circle (at -2.54 5.08) (size 4 4) (drill 4) (layers "*.Cu" "*.Mask"))
  (pad "" np_thru_hole circle (at 2.54 5.08) (size 1.7 1.7) (drill 1.7) (layers "*.Cu" "*.Mask"))
  (pad "1" thru_hole circle (at 0 0) (size 2.2 2.2) (drill 1.5) (layers "*.Cu" "*.Mask") (remove_unused_layers no) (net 1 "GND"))
  (pad "2" thru_hole circle (at -6.35 2.54) (size 2.2 2.2) (drill 1.5) (layers "*.Cu" "*.Mask") (remove_unused_layers no) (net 15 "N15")))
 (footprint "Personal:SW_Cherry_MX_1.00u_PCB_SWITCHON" (layer "F.Cu") (at 166.735 92.07)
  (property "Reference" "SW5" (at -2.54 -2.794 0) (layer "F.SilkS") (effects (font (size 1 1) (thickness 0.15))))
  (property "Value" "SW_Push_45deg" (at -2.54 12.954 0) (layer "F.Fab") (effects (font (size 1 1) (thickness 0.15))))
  (fp_line (start -9.525 -1.905) (end 4.445 -1.905) (stroke (width 0.12) (type solid)) (layer "F.SilkS"))
  (fp_line (start -9.525 12.065) (end -9.525 -1.905) (stroke (width 0.12) (type solid)) (layer "F.SilkS"))
  (fp_line (start 4.445 -1.905) (end 4.445 12.065) (stroke (width 0.12) (type solid)) (layer "F.SilkS"))
  (fp_line (start 4.445 12.065) (end -9.525 12.065) (stroke (width 0.12) (type solid)) (layer "F.SilkS"))
  (pad "" np_thru_hole circle (at -7.62 5.08) (size 1.7 1.7) (drill 1.7) (layers "*.Cu" "*.Mask"))
  (pad "" np_thru_hole circle (at -2.54 5.08) (size 4 4) (drill 4) (layers "*.Cu" "*.Mask"))
  (pad "" np_thru_hole circle (at 2.54 5.08) (size 1.7 1.7) (drill 1.7) (layers "*.Cu" "*.Mask"))
  (pad "1" thru_hole circle (at 0 0) (size 2.2 2.2) (drill 1.5) (layers "*.Cu" "*.Mask") (remove_unused_layers no) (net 1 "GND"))
  (pad "2" thru_hole circle (at -6.35 2.54) (size 2.2 2.2) (drill 1.5) (layers "*.Cu" "*.Mask") (remove_unused_layers no) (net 16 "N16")))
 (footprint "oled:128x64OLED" (layer "F.Cu") (at 140.8 50.025)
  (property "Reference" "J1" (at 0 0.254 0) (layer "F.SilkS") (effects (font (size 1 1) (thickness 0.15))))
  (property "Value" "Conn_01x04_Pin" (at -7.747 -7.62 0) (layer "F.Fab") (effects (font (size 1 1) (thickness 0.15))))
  (fp_line (start -13.4 -12.3) (end 14 -12.3) (stroke (width 0.12) (type solid)) (layer "F.SilkS"))
  (fp_line (start -13.4 15) (end -13.4 -12.3) (stroke (width 0.12) (type solid)) (layer "F.SilkS"))
  (fp_line (start -12.978 -9.005) (end 10.122 -9.005) (stroke (width 0.12) (type solid)) (layer "F.SilkS"))
  (fp_line (start -12.978 7.595) (end -12.978 -9.005) (stroke (width 0.12) (type solid)) (layer "F.SilkS"))
  (fp_line (start -4.699 -11.811) (end -4.699 -9.398) (stroke (width 0.12) (type solid)) (layer "F.SilkS"))
  (fp_line (start -4.699 -11.811) (end 5.08 -11.811) (stroke (width 0.12) (type solid)) (layer "F.SilkS"))
  (fp_line (start 5.08 -11.811) (end 5.08 -9.398) (stroke (width 0.12) (type solid)) (layer "F.SilkS"))
  (fp_line (start 5.08 -9.398) (end -4.699 -9.398) (stroke (width 0.12) (type solid)) (layer "F.SilkS"))
  (fp_line (start 10.122 -9.005) (end 13.208 -9.005) (stroke (width 0.12) (type solid)) (layer "F.SilkS"))
  (fp_line (start 10.122 7.595) (end -12.978 7.595) (stroke (width 0.12) (type solid)) (layer "F.SilkS"))
  (fp_line (start 10.122 7.595) (end 13.462 7.62) (stroke (width 0.12) (type solid)) (layer "F.SilkS"))
  (fp_line (start 13.462 -9.017) (end 13.208 -9.005) (stroke (width 0.12) (type solid)) (layer "F.SilkS"))
  (fp_line (start 13.462 7.62) (end 13.462 -9.017) (stroke (width 0.12) (type solid)) (layer "F.SilkS"))
  (fp_line (start 14 -12.3) (end 14 15) (stroke (width 0.12) (type solid)) (layer "F.SilkS"))
  (fp_line (start 14 15) (end -13.4 15) (stroke (width 0.12) (type solid)) (layer "F.SilkS"))
  (pad "1" thru_hole oval (at -3.62 -10.6 90) (size 2 1.6) (drill 1) (layers "*.Cu" "*.Mask") (remove_unused_layers no) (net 1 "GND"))
  (pad "2" thru_hole oval (at -1.08 -10.6 90) (size 2 1.6) (drill 1) (layers "*.Cu" "*.Mask") (remove_unused_layers no) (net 3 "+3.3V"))
  (pad "3" thru_hole oval (at 1.46 -10.6 90) (size 2 1.6) (drill 1) (layers "*.Cu" "*.Mask") (remove_unused_layers no) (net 14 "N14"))
  (pad "4" thru_hole oval (at 4 -10.6 90) (size 2 1.6) (drill 1) (layers "*.Cu" "*.Mask") (remove_unused_layers no) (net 13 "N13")))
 (gr_rect (start 100 34) (end 176.2 110.2) (stroke (width 0.05) (type solid)) (fill no) (layer "Edge.Cuts"))
 (segment (start 142.26 39.425) (end 138.7955 35.9605) (width 0.2) (layer "F.Cu") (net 14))
 (segment (start 118.793 35.9605) (end 105.03 49.7235) (width 0.2) (layer "F.Cu") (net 14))
 (segment (start 138.7955 35.9605) (end 118.793 35.9605) (width 0.2) (layer "F.Cu") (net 14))
 (segment (start 123.5385 39.5635) (end 120.27 39.5635) (width 0.2) (layer "F.Cu") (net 1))
 (segment (start 155.644 76.814) (end 155.644 73.85987) (width 0.2) (layer "F.Cu") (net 1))
 (segment (start 121.34763 39.5635) (end 121.105 39.5635) (width 0.2) (layer "F.Cu") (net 1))
 (segment (start 106.6 103.625) (end 119.207 91.018) (width 0.2) (layer "F.Cu") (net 1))
 (segment (start 121.34763 39.5635) (end 120.27 39.5635) (width 0.2) (layer "F.Cu") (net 1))
 (segment (start 135.3935 39.5635) (end 120.27 39.5635) (width 0.2) (layer "F.Cu") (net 1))
 (segment (start 147.68 61.279874) (end 125.963626 39.5635) (width 0.2) (layer "F.Cu") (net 1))
 (segment (start 156.945 78.115) (end 155.644 76.814) (width 0.2) (layer "F.Cu") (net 1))
 (segment (start 137.18 39.425) (end 121.2435 39.425) (width 0.2) (layer "F.Cu") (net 1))
 (segment (start 121.2435 39.425) (end 121.105 39.5635) (width 0.2) (layer "F.Cu") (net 1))
 (segment (start 166.735 92.07) (end 166.735 82.76) (width 0.2) (layer "F.Cu") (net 1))
 (segment (start 166.735 82.76) (end 123.5385 39.5635) (width 0.2) (layer "F.Cu") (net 1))
 (segment (start 155.644 73.85987) (end 121.34763 39.5635) (width 0.2) (layer "F.Cu") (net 1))
 (segment (start 128.645 42.244874) (end 125.963626 39.5635) (width 0.2) (layer "F.Cu") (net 1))
 (segment (start 119.207 91.018) (end 119.207 40.6265) (width 0.2) (layer "F.Cu") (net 1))
 (segment (start 128.645 73.035) (end 128.645 46.86087) (width 0.2) (layer "F.Cu") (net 1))
 (segment (start 128.645 92.085) (end 128.645 42.244874) (width 0.2) (layer "F.Cu") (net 1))
 (segment (start 119.207 40.6265) (end 120.27 39.5635) (width 0.2) (layer "F.Cu") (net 1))
 (segment (start 171.445 75.615) (end 135.3935 39.5635) (width 0.2) (layer "F.Cu") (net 1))
 (segment (start 125.963626 39.5635) (end 120.27 39.5635) (width 0.2) (layer "F.Cu") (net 1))
 (segment (start 128.645 46.86087) (end 121.34763 39.5635) (width 0.2) (layer "F.Cu") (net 1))
 (segment (start 147.68 92.07) (end 147.68 61.279874) (width 0.2) (layer "F.Cu") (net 1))
 (segment (start 117.6135 34.6) (end 105.03 47.1835) (width 0.2) (layer "F.Cu") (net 13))
 (segment (start 144.8 39.425) (end 139.975 34.6) (width 0.2) (layer "F.Cu") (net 13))
 (segment (start 139.975 34.6) (end 117.6135 34.6) (width 0.2) (layer "F.Cu") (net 13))
 (segment (start 120.20619 38.124) (end 118.225 40.10519) (width 0.2) (layer "F.Cu") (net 3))
 (segment (start 139.72 39.425) (end 138.419 38.124) (width 0.2) (layer "F.Cu") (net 3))
 (segment (start 118.225 40.10519) (end 118.225 42.175) (width 0.2) (layer "F.Cu") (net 3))
 (segment (start 138.419 38.124) (end 120.20619 38.124) (width 0.2) (layer "F.Cu") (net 3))
 (via (at 118.225 42.175) (size 0.6) (drill 0.3) (layers "F.Cu" "B.Cu") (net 3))
 (segment (start 106.6 63.625) (end 106.6 55.7735) (width 0.2) (layer "B.Cu") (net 3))
 (segment (start 118.225 42.175) (end 118.2965 42.1035) (width 0.2) (layer "B.Cu") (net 3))
 (segment (start 106.6 55.7735) (end 120.27 42.1035) (width 0.2) (layer "B.Cu") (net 3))
 (segment (start 118.2965 42.1035) (end 120.27 42.1035) (width 0.2) (layer "B.Cu") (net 3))
 (segment (start 122.295 75.575) (end 116.957595 75.575) (width 0.2) (layer "B.Cu") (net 7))
 (segment (start 105.03 63.647405) (end 105.03 52.2635) (width 0.2) (layer "B.Cu") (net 7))
 (segment (start 116.957595 75.575) (end 105.03 63.647405) (width 0.2) (layer "B.Cu") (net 7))
 (segment (start 141.345 73.3385) (end 120.27 52.2635) (width 0.2) (layer "B.Cu") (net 12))
 (segment (start 141.345 75.575) (end 141.345 73.3385) (width 0.2) (layer "B.Cu") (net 12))
 (segment (start 105.474 62.958) (end 118.607 49.825) (width 0.2) (layer "F.Cu") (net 11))
 (segment (start 122.295 94.625) (end 116.1671 94.625) (width 0.2) (layer "F.Cu") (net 11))
 (segment (start 116.1671 94.625) (end 107.726 103.0661) (width 0.2) (layer "F.Cu") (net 11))
 (segment (start 107.726 103.0661) (end 107.726 104.751) (width 0.2) (layer "F.Cu") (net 11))
 (segment (start 105.474 104.751) (end 105.474 62.958) (width 0.2) (layer "F.Cu") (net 11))
 (segment (start 107.726 104.751) (end 105.474 104.751) (width 0.2) (layer "F.Cu") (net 11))
 (via (at 118.607 49.825) (size 0.6) (drill 0.3) (layers "F.Cu" "B.Cu") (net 11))
 (segment (start 120.1685 49.825) (end 120.27 49.7235) (width 0.2) (layer "B.Cu") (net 11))
 (segment (start 118.607 49.825) (end 120.1685 49.825) (width 0.2) (layer "B.Cu") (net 11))
 (segment (start 141.33 94.61) (end 128.621586 94.61) (width 0.2) (layer "F.Cu") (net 15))
 (segment (start 123.353 89.341414) (end 123.353 78.614314) (width 0.2) (layer "F.Cu") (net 15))
 (segment (start 122.622 48.45787) (end 121.34763 47.1835) (width 0.2) (layer "F.Cu") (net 15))
 (segment (start 122.622 73.266686) (end 122.622 48.45787) (width 0.2) (layer "F.Cu") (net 15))
 (segment (start 120.894 74.994686) (end 122.622 73.266686) (width 0.2) (layer "F.Cu") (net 15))
 (segment (start 121.34763 47.1835) (end 120.27 47.1835) (width 0.2) (layer "F.Cu") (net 15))
 (segment (start 120.894 76.155314) (end 120.894 74.994686) (width 0.2) (layer "F.Cu") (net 15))
 (segment (start 123.353 78.614314) (end 120.894 76.155314) (width 0.2) (layer "F.Cu") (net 15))
 (segment (start 128.621586 94.61) (end 123.353 89.341414) (width 0.2) (layer "F.Cu") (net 15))
 (segment (start 130.046 92.665314) (end 129.225314 93.486) (width 0.2) (layer "F.Cu") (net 16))
 (segment (start 128.064686 93.486) (end 123.754 89.175314) (width 0.2) (layer "F.Cu") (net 16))
 (segment (start 123.754 89.175314) (end 123.754 47.04987) (width 0.2) (layer "F.Cu") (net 16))
 (segment (start 148.238686 94.61) (end 146.294 92.665314) (width 0.2) (layer "F.Cu") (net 16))
 (segment (start 146.294 92.665314) (end 130.046 92.665314) (width 0.2) (layer "F.Cu") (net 16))
 (segment (start 121.34763 44.6435) (end 120.27 44.6435) (width 0.2) (layer "F.Cu") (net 16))
 (segment (start 129.225314 93.486) (end 128.064686 93.486) (width 0.2) (layer "F.Cu") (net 16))
 (segment (start 160.385 94.61) (end 148.238686 94.61) (width 0.2) (layer "F.Cu") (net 16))
 (segment (start 123.754 47.04987) (end 121.34763 44.6435) (width 0.2) (layer "F.Cu") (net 16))
 (segment (start 156.945 75.615) (end 122.3705 41.0405) (width 0.2) (layer "B.Cu") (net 8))
 (segment (start 106.093 41.0405) (end 105.03 42.1035) (width 0.2) (layer "B.Cu") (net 8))
 (segment (start 122.3705 41.0405) (end 106.093 41.0405) (width 0.2) (layer "B.Cu") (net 8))
 (segment (start 102.277 36.622874) (end 102.939374 35.9605) (width 0.2) (layer "F.Cu") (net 10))
 (segment (start 104.034595 105.152) (end 102.277 103.394405) (width 0.2) (layer "F.Cu") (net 10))
 (segment (start 105.47031 35.9605) (end 106.0964 36.58659) (width 0.2) (layer "F.Cu") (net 10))
 (segment (start 171.445 80.615) (end 171.445 89.341314) (width 0.2) (layer "F.Cu") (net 10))
 (segment (start 102.939374 35.9605) (end 105.47031 35.9605) (width 0.2) (layer "F.Cu") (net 10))
 (segment (start 106.0964 43.5771) (end 105.03 44.6435) (width 0.2) (layer "F.Cu") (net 10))
 (segment (start 102.277 103.394405) (end 102.277 36.622874) (width 0.2) (layer "F.Cu") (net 10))
 (segment (start 152.832314 105.152) (end 104.034595 105.152) (width 0.2) (layer "F.Cu") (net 10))
 (segment (start 171.445 89.341314) (end 167.315314 93.471) (width 0.2) (layer "F.Cu") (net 10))
 (segment (start 164.513314 93.471) (end 152.832314 105.152) (width 0.2) (layer "F.Cu") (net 10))
 (segment (start 106.0964 36.58659) (end 106.0964 43.5771) (width 0.2) (layer "F.Cu") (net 10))
 (segment (start 167.315314 93.471) (end 164.513314 93.471) (width 0.2) (layer "F.Cu") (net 10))
 (segment (start 156.945 80.615) (end 121.430495 80.615) (width 0.2) (layer "B.Cu") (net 9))
 (segment (start 103.967 63.151505) (end 103.967 40.6265) (width 0.2) (layer "B.Cu") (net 9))
 (segment (start 121.430495 80.615) (end 103.967 63.151505) (width 0.2) (layer "B.Cu") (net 9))
 (segment (start 103.967 40.6265) (end 105.03 39.5635) (width 0.2) (layer "B.Cu") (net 9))
 (segment (start 102.678 102.203) (end 102.678 38.5405) (width 0.2) (layer "F.Cu") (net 2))
 (segment (start 102.678 38.5405) (end 104.195 37.0235) (width 0.2) (layer "F.Cu") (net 2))
 (segment (start 104.1 103.625) (end 102.678 102.203) (width 0.2) (layer "F.Cu") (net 2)))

